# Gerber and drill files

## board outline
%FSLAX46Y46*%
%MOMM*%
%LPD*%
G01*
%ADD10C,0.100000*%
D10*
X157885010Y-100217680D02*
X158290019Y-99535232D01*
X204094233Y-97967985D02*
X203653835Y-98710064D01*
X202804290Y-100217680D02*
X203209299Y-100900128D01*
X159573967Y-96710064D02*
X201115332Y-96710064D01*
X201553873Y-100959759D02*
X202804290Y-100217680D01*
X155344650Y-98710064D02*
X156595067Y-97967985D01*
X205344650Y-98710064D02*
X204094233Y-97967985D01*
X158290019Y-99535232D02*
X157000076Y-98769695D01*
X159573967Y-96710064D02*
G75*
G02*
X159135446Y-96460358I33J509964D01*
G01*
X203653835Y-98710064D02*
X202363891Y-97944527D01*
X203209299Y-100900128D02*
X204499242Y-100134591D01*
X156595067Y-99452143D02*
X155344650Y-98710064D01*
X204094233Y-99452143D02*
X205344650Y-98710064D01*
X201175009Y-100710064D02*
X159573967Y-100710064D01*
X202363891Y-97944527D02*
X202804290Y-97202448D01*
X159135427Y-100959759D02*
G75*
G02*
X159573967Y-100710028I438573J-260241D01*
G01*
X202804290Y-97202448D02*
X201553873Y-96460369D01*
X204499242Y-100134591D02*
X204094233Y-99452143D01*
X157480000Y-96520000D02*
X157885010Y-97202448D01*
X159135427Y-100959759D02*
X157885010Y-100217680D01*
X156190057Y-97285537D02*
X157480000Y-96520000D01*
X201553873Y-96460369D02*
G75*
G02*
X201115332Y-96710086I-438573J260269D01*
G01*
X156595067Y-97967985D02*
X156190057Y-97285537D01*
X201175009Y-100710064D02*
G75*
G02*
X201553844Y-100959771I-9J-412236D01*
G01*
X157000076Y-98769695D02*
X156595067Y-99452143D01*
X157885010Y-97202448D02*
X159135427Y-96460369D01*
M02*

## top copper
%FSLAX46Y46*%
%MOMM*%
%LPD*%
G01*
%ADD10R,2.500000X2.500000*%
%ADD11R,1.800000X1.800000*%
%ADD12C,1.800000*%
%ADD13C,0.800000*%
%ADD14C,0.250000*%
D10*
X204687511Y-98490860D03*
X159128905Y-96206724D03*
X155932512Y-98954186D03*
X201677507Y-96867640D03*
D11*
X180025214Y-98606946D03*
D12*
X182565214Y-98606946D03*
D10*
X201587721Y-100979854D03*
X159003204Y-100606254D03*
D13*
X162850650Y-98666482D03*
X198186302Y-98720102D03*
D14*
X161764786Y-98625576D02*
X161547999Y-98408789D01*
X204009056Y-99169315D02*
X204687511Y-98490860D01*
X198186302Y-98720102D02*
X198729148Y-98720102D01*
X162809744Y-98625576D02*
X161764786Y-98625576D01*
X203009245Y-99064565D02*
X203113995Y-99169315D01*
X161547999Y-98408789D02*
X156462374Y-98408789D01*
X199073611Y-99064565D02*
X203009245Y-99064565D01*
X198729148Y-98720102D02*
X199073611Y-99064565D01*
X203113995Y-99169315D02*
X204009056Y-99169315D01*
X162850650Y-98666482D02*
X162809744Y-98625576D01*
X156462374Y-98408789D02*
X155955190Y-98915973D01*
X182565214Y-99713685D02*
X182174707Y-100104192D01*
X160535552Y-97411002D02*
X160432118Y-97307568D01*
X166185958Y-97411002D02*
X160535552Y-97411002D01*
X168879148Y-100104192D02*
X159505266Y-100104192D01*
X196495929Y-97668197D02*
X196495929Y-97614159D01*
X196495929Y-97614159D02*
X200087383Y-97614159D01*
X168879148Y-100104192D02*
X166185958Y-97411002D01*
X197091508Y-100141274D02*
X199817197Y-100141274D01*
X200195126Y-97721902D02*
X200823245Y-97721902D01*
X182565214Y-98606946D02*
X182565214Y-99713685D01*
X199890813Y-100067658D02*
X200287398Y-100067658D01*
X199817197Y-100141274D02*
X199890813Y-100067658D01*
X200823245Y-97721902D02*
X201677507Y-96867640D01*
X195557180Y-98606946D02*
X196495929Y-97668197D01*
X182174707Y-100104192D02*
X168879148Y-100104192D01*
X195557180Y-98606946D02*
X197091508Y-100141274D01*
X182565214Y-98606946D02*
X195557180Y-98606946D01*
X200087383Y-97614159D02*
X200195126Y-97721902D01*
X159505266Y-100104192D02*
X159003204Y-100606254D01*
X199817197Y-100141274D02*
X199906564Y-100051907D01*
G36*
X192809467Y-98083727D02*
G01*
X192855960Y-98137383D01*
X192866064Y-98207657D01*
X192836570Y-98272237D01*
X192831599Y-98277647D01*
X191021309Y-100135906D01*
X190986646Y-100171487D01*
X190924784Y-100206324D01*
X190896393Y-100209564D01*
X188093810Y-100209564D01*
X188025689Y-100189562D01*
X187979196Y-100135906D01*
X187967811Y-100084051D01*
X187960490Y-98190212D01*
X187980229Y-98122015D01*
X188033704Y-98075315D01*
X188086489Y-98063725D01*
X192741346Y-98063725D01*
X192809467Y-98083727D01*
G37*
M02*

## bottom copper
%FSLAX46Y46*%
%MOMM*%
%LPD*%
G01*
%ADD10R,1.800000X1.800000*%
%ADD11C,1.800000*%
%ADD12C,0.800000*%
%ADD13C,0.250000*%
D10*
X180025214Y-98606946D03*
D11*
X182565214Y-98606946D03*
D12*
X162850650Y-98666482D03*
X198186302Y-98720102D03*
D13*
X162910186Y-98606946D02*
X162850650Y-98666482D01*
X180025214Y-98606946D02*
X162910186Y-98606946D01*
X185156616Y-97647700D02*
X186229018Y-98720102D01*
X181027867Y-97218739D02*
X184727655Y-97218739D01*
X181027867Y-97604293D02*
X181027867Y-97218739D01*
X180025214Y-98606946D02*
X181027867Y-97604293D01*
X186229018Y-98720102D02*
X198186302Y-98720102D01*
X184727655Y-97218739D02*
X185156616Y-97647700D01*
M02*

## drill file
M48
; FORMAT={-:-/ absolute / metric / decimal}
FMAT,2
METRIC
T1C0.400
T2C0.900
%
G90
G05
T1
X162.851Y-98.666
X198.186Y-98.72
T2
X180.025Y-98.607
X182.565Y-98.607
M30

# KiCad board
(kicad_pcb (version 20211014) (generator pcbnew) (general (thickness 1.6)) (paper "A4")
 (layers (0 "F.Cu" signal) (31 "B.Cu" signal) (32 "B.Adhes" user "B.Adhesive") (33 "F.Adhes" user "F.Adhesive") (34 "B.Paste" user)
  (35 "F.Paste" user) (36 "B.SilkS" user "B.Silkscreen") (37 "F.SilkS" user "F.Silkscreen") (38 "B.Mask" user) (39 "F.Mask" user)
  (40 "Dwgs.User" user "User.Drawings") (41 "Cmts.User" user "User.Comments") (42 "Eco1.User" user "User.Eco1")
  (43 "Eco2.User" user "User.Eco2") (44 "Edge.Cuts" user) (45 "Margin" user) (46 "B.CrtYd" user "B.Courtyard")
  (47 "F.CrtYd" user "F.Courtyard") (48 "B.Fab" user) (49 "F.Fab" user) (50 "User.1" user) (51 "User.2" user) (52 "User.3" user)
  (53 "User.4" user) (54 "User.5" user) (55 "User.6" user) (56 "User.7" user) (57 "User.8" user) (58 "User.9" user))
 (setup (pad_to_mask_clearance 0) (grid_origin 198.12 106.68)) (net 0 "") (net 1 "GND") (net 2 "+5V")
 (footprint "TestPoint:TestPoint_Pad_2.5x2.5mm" (layer "F.Cu") (at 204.687511 98.49086)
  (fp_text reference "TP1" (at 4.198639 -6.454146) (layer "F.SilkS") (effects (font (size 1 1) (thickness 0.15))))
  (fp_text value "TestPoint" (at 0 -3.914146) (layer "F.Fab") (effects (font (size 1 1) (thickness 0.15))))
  (pad "1" smd rect (at 0 0) (size 2.5 2.5) (layers "F.Cu" "F.Mask") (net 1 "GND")))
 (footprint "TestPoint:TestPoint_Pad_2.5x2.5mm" (layer "F.Cu") (at 159.128905 96.206724)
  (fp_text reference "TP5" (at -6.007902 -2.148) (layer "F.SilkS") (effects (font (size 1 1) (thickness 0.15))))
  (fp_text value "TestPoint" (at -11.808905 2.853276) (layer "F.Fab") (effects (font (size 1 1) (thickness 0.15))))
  (pad "1" smd rect (at 0 0) (size 2.5 2.5) (layers "F.Cu" "F.Mask") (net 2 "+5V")))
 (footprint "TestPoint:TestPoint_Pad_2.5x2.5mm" (layer "F.Cu") (at 155.932512 98.954186)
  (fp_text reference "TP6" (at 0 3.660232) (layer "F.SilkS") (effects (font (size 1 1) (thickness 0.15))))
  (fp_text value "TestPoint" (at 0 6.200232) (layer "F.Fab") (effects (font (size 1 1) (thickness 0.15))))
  (pad "1" smd rect (at 0 0) (size 2.5 2.5) (layers "F.Cu" "F.Mask") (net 1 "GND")))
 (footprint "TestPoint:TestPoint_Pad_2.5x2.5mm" (layer "F.Cu") (at 201.677507 96.86764)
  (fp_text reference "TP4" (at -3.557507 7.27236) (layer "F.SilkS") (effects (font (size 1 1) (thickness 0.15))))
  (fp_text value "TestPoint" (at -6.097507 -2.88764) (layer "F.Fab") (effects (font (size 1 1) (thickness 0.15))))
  (pad "1" smd rect (at 0 0) (size 2.5 2.5) (layers "F.Cu" "F.Mask") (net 2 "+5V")))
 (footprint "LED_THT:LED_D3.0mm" (layer "F.Cu") (at 180.025214 98.606946)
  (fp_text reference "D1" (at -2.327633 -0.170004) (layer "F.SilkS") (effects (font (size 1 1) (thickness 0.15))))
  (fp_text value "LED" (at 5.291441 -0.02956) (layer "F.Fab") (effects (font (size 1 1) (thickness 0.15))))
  (pad "1" thru_hole rect (at 0 0) (size 1.8 1.8) (drill 0.9) (layers *.Cu *.Mask) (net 1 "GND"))
  (pad "2" thru_hole circle (at 2.54 0) (size 1.8 1.8) (drill 0.9) (layers *.Cu *.Mask) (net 2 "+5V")))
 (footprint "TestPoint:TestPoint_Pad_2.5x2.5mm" (layer "F.Cu") (at 201.587721 100.979854)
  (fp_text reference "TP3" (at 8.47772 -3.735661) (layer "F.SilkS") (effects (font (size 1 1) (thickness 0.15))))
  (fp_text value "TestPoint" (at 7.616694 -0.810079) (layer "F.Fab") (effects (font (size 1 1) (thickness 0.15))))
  (pad "1" smd rect (at 0 0) (size 2.5 2.5) (layers "F.Cu" "F.Mask") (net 2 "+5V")))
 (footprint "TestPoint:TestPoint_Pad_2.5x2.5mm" (layer "F.Cu") (at 159.003204 100.606254)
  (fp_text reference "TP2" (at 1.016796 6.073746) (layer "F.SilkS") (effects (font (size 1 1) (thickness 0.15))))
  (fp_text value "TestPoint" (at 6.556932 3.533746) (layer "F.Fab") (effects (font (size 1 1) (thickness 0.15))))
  (pad "1" smd rect (at 0 0) (size 2.5 2.5) (layers "F.Cu" "F.Mask") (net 2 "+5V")))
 (gr_line (start 157.88501 100.21768) (end 158.290019 99.535232) (layer "Edge.Cuts") (width 0.1))
 (gr_line (start 204.094233 97.967985) (end 203.653835 98.710064) (layer "Edge.Cuts") (width 0.1))
 (gr_line (start 202.80429 100.21768) (end 203.209299 100.900128) (layer "Edge.Cuts") (width 0.1))
 (gr_line (start 159.573967 96.710064) (end 201.115332 96.710064) (layer "Edge.Cuts") (width 0.1))
 (gr_line (start 201.553873 100.959759) (end 202.80429 100.21768) (layer "Edge.Cuts") (width 0.1))
 (gr_line (start 155.34465 98.710064) (end 156.595067 97.967985) (layer "Edge.Cuts") (width 0.1))
 (gr_line (start 205.34465 98.710064) (end 204.094233 97.967985) (layer "Edge.Cuts") (width 0.1))
 (gr_line (start 158.290019 99.535232) (end 157.000076 98.769695) (layer "Edge.Cuts") (width 0.1))
 (gr_arc (start 159.573967 96.710064) (mid 159.321645 96.643265) (end 159.135427 96.460369) (layer "Edge.Cuts") (width 0.1))
 (gr_line (start 203.653835 98.710064) (end 202.363891 97.944527) (layer "Edge.Cuts") (width 0.1))
 (gr_line (start 203.209299 100.900128) (end 204.499242 100.134591) (layer "Edge.Cuts") (width 0.1))
 (gr_line (start 156.595067 99.452143) (end 155.34465 98.710064) (layer "Edge.Cuts") (width 0.1))
 (gr_line (start 204.094233 99.452143) (end 205.34465 98.710064) (layer "Edge.Cuts") (width 0.1))
 (gr_line (start 201.175009 100.710064) (end 159.573967 100.710064) (layer "Edge.Cuts") (width 0.1))
 (gr_line (start 202.363891 97.944527) (end 202.80429 97.202448) (layer "Edge.Cuts") (width 0.1))
 (gr_arc (start 159.135427 100.959759) (mid 159.321645 100.776863) (end 159.573967 100.710064) (layer "Edge.Cuts") (width 0.1))
 (gr_line (start 202.80429 97.202448) (end 201.553873 96.460369) (layer "Edge.Cuts") (width 0.1))
 (gr_line (start 204.499242 100.134591) (end 204.094233 99.452143) (layer "Edge.Cuts") (width 0.1))
 (gr_line (start 157.48 96.52) (end 157.88501 97.202448) (layer "Edge.Cuts") (width 0.1))
 (gr_line (start 159.135427 100.959759) (end 157.88501 100.21768) (layer "Edge.Cuts") (width 0.1))
 (gr_line (start 156.190057 97.285537) (end 157.48 96.52) (layer "Edge.Cuts") (width 0.1))
 (gr_arc (start 201.553873 96.460369) (mid 201.367654 96.643265) (end 201.115332 96.710064) (layer "Edge.Cuts") (width 0.1))
 (gr_line (start 156.595067 97.967985) (end 156.190057 97.285537) (layer "Edge.Cuts") (width 0.1))
 (gr_arc (start 201.175009 100.710064) (mid 201.401882 100.778102) (end 201.553873 100.959759) (layer "Edge.Cuts") (width 0.1))
 (gr_line (start 157.000076 98.769695) (end 156.595067 99.452143) (layer "Edge.Cuts") (width 0.1))
 (gr_line (start 157.88501 97.202448) (end 159.135427 96.460369) (layer "Edge.Cuts") (width 0.1))
 (segment (start 161.764786 98.625576) (end 161.547999 98.408789) (width 0.25) (layer "F.Cu") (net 1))
 (segment (start 204.009056 99.169315) (end 204.687511 98.49086) (width 0.25) (layer "F.Cu") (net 1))
 (segment (start 198.186302 98.720102) (end 198.729148 98.720102) (width 0.25) (layer "F.Cu") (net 1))
 (segment (start 162.809744 98.625576) (end 161.764786 98.625576) (width 0.25) (layer "F.Cu") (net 1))
 (segment (start 203.009245 99.064565) (end 203.113995 99.169315) (width 0.25) (layer "F.Cu") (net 1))
 (segment (start 161.547999 98.408789) (end 156.462374 98.408789) (width 0.25) (layer "F.Cu") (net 1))
 (segment (start 199.073611 99.064565) (end 203.009245 99.064565) (width 0.25) (layer "F.Cu") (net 1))
 (segment (start 198.729148 98.720102) (end 199.073611 99.064565) (width 0.25) (layer "F.Cu") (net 1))
 (segment (start 203.113995 99.169315) (end 204.009056 99.169315) (width 0.25) (layer "F.Cu") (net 1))
 (segment (start 162.85065 98.666482) (end 162.809744 98.625576) (width 0.25) (layer "F.Cu") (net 1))
 (segment (start 156.462374 98.408789) (end 155.95519 98.915973) (width 0.25) (layer "F.Cu") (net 1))
 (via (at 162.85065 98.666482) (size 0.8) (drill 0.4) (layers "F.Cu" "B.Cu") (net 1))
 (via (at 198.186302 98.720102) (size 0.8) (drill 0.4) (layers "F.Cu" "B.Cu") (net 1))
 (segment (start 162.910186 98.606946) (end 162.85065 98.666482) (width 0.25) (layer "B.Cu") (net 1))
 (segment (start 180.025214 98.606946) (end 162.910186 98.606946) (width 0.25) (layer "B.Cu") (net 1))
 (segment (start 185.156616 97.6477) (end 186.229018 98.720102) (width 0.25) (layer "B.Cu") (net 1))
 (segment (start 181.027867 97.218739) (end 184.727655 97.218739) (width 0.25) (layer "B.Cu") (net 1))
 (segment (start 181.027867 97.604293) (end 181.027867 97.218739) (width 0.25) (layer "B.Cu") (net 1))
 (segment (start 180.025214 98.606946) (end 181.027867 97.604293) (width 0.25) (layer "B.Cu") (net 1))
 (segment (start 186.229018 98.720102) (end 198.186302 98.720102) (width 0.25) (layer "B.Cu") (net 1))
 (segment (start 184.727655 97.218739) (end 185.156616 97.6477) (width 0.25) (layer "B.Cu") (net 1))
 (segment (start 182.565214 99.713685) (end 182.174707 100.104192) (width 0.25) (layer "F.Cu") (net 2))
 (segment (start 160.535552 97.411002) (end 160.432118 97.307568) (width 0.25) (layer "F.Cu") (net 2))
 (segment (start 166.185958 97.411002) (end 160.535552 97.411002) (width 0.25) (layer "F.Cu") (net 2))
 (segment (start 168.879148 100.104192) (end 159.505266 100.104192) (width 0.25) (layer "F.Cu") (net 2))
 (segment (start 196.495929 97.668197) (end 196.495929 97.614159) (width 0.25) (layer "F.Cu") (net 2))
 (segment (start 196.495929 97.614159) (end 200.087383 97.614159) (width 0.25) (layer "F.Cu") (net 2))
 (segment (start 168.879148 100.104192) (end 166.185958 97.411002) (width 0.25) (layer "F.Cu") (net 2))
 (segment (start 197.091508 100.141274) (end 199.817197 100.141274) (width 0.25) (layer "F.Cu") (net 2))
 (segment (start 200.195126 97.721902) (end 200.823245 97.721902) (width 0.25) (layer "F.Cu") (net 2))
 (segment (start 182.565214 98.606946) (end 182.565214 99.713685) (width 0.25) (layer "F.Cu") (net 2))
 (segment (start 199.890813 100.067658) (end 200.287398 100.067658) (width 0.25) (layer "F.Cu") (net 2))
 (segment (start 199.817197 100.141274) (end 199.890813 100.067658) (width 0.25) (layer "F.Cu") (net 2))
 (segment (start 200.823245 97.721902) (end 201.677507 96.86764) (width 0.25) (layer "F.Cu") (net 2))
 (segment (start 195.55718 98.606946) (end 196.495929 97.668197) (width 0.25) (layer "F.Cu") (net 2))
 (segment (start 182.174707 100.104192) (end 168.879148 100.104192) (width 0.25) (layer "F.Cu") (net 2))
 (segment (start 195.55718 98.606946) (end 197.091508 100.141274) (width 0.25) (layer "F.Cu") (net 2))
 (segment (start 182.565214 98.606946) (end 195.55718 98.606946) (width 0.25) (layer "F.Cu") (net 2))
 (segment (start 200.087383 97.614159) (end 200.195126 97.721902) (width 0.25) (layer "F.Cu") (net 2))
 (segment (start 159.505266 100.104192) (end 159.003204 100.606254) (width 0.25) (layer "F.Cu") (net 2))
 (segment (start 199.817197 100.141274) (end 199.906564 100.051907) (width 0.25) (layer "F.Cu") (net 2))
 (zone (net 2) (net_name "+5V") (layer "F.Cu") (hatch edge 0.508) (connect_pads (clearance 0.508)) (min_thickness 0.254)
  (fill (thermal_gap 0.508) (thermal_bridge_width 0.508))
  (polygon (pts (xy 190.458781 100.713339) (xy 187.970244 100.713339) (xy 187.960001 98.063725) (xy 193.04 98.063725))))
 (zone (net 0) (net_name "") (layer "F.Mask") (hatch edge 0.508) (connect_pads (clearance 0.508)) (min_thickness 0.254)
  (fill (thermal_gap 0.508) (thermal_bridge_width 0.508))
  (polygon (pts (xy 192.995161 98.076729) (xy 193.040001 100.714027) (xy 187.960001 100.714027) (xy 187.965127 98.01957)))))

